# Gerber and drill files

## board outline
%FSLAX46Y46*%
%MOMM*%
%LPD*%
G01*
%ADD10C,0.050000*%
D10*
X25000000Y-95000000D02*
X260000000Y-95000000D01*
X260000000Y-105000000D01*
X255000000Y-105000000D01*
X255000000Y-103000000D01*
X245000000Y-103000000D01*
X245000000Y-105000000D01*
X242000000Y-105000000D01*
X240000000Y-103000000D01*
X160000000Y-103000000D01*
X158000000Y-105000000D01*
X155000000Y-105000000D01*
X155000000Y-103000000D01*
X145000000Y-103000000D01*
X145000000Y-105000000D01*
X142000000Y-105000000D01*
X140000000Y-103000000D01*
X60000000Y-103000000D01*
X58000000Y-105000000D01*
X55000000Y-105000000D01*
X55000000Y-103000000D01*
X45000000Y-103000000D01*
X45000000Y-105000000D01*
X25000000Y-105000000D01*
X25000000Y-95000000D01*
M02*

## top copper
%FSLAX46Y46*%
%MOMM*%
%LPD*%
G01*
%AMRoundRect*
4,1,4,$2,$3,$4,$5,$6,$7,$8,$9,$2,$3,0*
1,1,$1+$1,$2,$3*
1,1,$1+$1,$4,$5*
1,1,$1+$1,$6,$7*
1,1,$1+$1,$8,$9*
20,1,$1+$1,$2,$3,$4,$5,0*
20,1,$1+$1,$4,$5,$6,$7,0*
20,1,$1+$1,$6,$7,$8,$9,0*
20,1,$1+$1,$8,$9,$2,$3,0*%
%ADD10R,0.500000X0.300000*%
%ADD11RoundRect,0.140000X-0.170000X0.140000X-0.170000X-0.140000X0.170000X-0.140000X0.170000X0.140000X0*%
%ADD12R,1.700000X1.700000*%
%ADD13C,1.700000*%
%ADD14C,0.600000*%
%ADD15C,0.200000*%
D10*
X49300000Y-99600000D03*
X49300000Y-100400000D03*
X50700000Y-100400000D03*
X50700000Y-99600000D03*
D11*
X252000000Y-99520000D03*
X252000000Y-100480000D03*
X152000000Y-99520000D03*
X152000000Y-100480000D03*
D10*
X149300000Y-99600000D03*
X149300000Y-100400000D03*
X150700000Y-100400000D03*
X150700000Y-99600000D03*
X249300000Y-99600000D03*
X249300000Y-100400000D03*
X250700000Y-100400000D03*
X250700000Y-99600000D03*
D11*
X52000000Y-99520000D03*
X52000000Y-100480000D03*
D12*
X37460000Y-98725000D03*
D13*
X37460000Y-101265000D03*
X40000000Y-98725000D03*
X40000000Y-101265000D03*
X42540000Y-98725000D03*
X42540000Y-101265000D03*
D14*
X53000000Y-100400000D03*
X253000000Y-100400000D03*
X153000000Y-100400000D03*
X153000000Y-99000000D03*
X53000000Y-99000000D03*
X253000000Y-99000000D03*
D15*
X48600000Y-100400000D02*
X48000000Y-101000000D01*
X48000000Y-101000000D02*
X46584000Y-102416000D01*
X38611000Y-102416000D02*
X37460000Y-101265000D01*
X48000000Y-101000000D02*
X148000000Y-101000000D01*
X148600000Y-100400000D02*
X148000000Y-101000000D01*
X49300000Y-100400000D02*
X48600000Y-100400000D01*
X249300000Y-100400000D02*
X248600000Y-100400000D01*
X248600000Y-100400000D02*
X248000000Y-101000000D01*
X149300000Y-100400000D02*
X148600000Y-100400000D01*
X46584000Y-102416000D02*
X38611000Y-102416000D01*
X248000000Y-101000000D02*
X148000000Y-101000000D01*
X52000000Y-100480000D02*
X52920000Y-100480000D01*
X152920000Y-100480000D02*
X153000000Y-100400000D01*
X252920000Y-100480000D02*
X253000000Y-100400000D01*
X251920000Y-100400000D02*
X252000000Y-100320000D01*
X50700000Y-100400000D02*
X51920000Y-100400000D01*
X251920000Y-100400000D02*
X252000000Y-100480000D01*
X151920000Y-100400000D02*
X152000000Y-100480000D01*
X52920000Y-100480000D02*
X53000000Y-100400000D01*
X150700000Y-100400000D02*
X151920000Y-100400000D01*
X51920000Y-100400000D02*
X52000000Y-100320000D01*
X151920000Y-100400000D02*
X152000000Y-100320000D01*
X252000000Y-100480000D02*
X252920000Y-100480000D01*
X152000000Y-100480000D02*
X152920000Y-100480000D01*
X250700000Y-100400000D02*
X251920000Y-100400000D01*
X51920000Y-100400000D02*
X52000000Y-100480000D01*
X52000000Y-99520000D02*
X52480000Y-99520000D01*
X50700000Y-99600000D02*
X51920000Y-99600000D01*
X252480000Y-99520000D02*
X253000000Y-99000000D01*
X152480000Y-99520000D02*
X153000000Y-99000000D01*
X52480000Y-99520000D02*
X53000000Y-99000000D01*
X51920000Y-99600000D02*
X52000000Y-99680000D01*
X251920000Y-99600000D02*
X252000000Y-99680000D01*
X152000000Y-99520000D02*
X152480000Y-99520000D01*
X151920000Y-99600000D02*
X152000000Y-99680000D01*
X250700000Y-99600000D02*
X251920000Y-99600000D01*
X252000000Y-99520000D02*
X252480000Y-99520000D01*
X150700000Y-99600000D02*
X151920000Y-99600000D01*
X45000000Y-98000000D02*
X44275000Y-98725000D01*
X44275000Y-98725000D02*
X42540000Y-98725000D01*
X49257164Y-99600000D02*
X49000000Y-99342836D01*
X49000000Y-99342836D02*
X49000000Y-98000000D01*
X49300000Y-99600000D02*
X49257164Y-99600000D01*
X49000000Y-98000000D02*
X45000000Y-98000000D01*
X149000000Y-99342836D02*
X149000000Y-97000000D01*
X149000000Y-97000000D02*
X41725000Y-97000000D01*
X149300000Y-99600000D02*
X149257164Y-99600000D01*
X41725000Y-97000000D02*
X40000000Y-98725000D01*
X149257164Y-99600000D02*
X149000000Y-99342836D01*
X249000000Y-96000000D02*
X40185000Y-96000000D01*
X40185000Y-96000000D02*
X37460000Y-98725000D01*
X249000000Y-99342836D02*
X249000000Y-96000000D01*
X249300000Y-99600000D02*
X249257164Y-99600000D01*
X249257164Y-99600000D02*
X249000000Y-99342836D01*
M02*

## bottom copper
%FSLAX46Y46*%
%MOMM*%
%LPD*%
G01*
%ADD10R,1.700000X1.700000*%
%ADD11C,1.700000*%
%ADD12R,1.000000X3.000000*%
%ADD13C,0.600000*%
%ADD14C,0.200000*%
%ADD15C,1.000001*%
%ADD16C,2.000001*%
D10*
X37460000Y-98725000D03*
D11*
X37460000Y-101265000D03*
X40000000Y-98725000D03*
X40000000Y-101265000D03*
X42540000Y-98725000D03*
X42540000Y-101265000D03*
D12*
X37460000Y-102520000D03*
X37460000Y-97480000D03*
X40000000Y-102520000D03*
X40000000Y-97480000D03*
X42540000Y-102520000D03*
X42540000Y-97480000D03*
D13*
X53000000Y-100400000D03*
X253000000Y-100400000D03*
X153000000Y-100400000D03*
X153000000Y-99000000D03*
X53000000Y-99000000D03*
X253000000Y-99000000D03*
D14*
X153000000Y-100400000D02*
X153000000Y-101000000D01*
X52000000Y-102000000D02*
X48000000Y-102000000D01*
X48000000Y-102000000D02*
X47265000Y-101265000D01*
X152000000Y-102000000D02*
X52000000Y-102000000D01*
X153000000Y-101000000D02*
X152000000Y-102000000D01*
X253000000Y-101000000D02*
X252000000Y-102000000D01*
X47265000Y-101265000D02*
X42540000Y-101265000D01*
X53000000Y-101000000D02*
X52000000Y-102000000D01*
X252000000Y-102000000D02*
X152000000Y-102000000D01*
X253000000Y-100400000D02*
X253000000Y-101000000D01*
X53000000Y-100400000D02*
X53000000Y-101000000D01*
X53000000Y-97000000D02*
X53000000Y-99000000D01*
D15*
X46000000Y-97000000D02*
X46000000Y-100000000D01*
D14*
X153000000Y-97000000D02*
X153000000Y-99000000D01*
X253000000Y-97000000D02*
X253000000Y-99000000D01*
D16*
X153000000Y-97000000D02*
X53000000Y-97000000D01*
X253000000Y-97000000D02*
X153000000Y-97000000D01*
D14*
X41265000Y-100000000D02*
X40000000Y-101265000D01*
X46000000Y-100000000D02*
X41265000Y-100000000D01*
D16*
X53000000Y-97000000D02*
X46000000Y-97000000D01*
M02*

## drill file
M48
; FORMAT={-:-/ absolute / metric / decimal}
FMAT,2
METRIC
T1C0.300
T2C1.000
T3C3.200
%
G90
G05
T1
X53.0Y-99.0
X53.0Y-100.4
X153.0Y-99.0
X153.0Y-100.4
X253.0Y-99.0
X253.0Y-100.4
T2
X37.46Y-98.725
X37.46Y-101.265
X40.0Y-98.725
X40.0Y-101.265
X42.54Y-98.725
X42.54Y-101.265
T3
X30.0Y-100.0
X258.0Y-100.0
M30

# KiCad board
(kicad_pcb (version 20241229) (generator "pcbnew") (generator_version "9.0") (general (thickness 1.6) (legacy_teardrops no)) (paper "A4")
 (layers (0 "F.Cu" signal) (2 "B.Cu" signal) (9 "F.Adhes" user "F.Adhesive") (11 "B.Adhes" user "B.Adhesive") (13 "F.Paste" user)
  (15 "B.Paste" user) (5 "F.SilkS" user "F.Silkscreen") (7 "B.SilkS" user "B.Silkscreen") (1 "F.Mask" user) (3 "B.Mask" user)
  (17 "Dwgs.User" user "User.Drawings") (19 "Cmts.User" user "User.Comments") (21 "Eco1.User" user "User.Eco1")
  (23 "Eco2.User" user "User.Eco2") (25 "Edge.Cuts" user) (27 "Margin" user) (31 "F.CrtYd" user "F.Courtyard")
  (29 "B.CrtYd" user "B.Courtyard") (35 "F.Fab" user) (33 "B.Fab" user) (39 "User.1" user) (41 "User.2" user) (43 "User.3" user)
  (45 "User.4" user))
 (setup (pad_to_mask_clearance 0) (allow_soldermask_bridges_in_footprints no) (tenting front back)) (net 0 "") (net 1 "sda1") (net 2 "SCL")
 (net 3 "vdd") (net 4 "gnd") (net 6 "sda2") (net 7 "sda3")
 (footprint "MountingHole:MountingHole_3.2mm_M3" (layer "F.Cu") (at 258 100)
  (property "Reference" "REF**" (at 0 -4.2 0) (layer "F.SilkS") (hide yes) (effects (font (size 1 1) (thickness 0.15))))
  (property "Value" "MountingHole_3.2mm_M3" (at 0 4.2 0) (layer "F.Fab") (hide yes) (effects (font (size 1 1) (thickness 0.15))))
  (pad "" np_thru_hole circle (at 0 0) (size 3.2 3.2) (drill 3.2) (layers "*.Cu" "*.Mask")))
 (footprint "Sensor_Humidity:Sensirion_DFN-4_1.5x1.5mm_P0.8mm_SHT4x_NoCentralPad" (layer "F.Cu") (at 50 100)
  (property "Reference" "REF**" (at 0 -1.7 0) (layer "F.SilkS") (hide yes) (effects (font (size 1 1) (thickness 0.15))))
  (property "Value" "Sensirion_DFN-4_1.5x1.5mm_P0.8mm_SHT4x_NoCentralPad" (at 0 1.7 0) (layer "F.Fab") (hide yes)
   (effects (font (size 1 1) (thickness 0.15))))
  (pad "1" smd rect (at -0.7 -0.4) (size 0.5 0.3) (layers "F.Cu" "F.Mask" "F.Paste") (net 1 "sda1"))
  (pad "2" smd rect (at -0.7 0.4) (size 0.5 0.3) (layers "F.Cu" "F.Mask" "F.Paste") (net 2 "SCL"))
  (pad "3" smd rect (at 0.7 0.4) (size 0.5 0.3) (layers "F.Cu" "F.Mask" "F.Paste") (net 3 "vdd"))
  (pad "4" smd rect (at 0.7 -0.4) (size 0.5 0.3) (layers "F.Cu" "F.Mask" "F.Paste") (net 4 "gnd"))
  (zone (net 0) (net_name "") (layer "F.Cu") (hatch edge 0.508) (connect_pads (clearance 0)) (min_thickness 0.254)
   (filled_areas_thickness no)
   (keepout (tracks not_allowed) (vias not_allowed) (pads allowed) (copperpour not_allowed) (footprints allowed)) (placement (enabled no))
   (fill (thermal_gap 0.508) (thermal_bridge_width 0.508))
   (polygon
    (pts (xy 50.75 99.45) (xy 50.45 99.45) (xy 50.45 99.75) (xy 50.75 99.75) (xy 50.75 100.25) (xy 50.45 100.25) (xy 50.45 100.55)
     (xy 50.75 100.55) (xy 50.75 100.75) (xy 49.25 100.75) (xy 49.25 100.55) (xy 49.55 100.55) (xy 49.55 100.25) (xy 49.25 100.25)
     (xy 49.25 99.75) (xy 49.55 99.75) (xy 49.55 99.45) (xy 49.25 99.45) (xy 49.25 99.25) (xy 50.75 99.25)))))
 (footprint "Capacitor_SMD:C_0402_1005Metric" (layer "F.Cu") (at 252 100 -90)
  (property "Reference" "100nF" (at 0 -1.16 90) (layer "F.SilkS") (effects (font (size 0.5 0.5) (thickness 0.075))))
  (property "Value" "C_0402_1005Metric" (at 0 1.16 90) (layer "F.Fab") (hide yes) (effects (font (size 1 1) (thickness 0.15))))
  (pad "1" smd roundrect (at -0.48 0 270) (size 0.56 0.62) (layers "F.Cu" "F.Mask" "F.Paste") (roundrect_rratio 0.25) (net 4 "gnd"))
  (pad "2" smd roundrect (at 0.48 0 270) (size 0.56 0.62) (layers "F.Cu" "F.Mask" "F.Paste") (roundrect_rratio 0.25) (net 3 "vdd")))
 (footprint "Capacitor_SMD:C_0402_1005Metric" (layer "F.Cu") (at 152 100 -90)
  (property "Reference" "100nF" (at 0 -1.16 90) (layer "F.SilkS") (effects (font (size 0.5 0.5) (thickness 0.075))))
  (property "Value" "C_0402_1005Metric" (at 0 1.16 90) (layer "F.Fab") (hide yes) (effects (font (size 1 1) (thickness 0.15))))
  (pad "1" smd roundrect (at -0.48 0 270) (size 0.56 0.62) (layers "F.Cu" "F.Mask" "F.Paste") (roundrect_rratio 0.25) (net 4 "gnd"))
  (pad "2" smd roundrect (at 0.48 0 270) (size 0.56 0.62) (layers "F.Cu" "F.Mask" "F.Paste") (roundrect_rratio 0.25) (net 3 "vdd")))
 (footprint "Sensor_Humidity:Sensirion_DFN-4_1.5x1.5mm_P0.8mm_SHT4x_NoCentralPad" (layer "F.Cu") (at 150 100)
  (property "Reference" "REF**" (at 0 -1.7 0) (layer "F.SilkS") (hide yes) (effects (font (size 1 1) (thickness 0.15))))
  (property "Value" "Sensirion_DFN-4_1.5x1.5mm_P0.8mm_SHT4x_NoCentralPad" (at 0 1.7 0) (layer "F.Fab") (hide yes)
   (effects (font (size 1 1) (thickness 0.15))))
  (pad "1" smd rect (at -0.7 -0.4) (size 0.5 0.3) (layers "F.Cu" "F.Mask" "F.Paste") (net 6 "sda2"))
  (pad "2" smd rect (at -0.7 0.4) (size 0.5 0.3) (layers "F.Cu" "F.Mask" "F.Paste") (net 2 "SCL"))
  (pad "3" smd rect (at 0.7 0.4) (size 0.5 0.3) (layers "F.Cu" "F.Mask" "F.Paste"))
  (pad "4" smd rect (at 0.7 -0.4) (size 0.5 0.3) (layers "F.Cu" "F.Mask" "F.Paste"))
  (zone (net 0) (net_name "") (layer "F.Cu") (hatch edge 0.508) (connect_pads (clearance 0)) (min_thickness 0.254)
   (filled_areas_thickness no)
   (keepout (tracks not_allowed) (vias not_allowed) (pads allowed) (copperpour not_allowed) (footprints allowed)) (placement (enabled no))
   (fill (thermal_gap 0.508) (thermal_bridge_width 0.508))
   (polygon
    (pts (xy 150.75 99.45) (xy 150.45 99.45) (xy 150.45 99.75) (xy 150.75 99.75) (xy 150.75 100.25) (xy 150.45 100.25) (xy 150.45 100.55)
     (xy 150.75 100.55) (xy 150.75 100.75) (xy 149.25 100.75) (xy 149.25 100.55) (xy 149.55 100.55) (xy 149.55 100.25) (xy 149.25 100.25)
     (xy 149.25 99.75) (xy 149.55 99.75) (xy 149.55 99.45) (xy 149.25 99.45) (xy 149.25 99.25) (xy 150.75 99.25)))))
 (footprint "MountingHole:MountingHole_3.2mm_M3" (layer "F.Cu") (at 30 100)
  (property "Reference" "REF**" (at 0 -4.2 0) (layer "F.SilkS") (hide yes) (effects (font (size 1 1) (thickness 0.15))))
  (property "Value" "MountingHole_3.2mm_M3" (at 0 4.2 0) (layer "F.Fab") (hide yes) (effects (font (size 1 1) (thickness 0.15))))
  (pad "" np_thru_hole circle (at 0 0) (size 3.2 3.2) (drill 3.2) (layers "*.Cu" "*.Mask")))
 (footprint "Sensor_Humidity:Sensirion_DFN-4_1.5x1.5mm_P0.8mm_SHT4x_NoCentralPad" (layer "F.Cu") (at 250 100)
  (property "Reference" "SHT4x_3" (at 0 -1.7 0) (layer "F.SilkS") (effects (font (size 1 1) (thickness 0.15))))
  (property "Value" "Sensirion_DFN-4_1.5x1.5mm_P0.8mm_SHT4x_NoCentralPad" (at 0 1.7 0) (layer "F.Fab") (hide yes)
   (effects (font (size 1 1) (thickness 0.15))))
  (pad "1" smd rect (at -0.7 -0.4) (size 0.5 0.3) (layers "F.Cu" "F.Mask" "F.Paste") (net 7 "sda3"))
  (pad "2" smd rect (at -0.7 0.4) (size 0.5 0.3) (layers "F.Cu" "F.Mask" "F.Paste") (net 2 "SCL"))
  (pad "3" smd rect (at 0.7 0.4) (size 0.5 0.3) (layers "F.Cu" "F.Mask" "F.Paste") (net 3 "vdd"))
  (pad "4" smd rect (at 0.7 -0.4) (size 0.5 0.3) (layers "F.Cu" "F.Mask" "F.Paste"))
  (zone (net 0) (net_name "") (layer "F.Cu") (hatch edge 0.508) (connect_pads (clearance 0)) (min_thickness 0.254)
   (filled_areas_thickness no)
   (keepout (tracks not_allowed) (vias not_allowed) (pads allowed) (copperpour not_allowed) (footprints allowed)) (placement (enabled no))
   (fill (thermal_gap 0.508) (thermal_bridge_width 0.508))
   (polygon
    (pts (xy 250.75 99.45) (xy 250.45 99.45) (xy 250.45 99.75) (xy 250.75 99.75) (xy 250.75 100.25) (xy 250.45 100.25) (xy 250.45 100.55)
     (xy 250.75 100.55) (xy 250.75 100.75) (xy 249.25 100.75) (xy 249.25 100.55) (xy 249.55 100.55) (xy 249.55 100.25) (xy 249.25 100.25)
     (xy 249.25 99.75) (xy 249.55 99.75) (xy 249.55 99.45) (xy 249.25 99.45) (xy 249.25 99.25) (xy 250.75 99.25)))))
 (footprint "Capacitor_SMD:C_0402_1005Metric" (layer "F.Cu") (at 52 100 -90)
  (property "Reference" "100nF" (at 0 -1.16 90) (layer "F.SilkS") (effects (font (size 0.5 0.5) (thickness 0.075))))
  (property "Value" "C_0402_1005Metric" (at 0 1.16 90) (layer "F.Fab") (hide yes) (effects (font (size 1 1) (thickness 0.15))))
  (pad "1" smd roundrect (at -0.48 0 270) (size 0.56 0.62) (layers "F.Cu" "F.Mask" "F.Paste") (roundrect_rratio 0.25) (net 4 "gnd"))
  (pad "2" smd roundrect (at 0.48 0 270) (size 0.56 0.62) (layers "F.Cu" "F.Mask" "F.Paste") (roundrect_rratio 0.25) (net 3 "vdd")))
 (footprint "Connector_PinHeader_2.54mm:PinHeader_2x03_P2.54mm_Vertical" (layer "B.Cu") (at 37.46 98.725 -90)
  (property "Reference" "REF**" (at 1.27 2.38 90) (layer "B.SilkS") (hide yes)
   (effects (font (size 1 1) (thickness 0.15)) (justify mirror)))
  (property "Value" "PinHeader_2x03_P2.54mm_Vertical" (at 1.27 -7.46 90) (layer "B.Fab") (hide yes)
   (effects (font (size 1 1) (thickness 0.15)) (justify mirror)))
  (pad "1" thru_hole rect (at 0 0 270) (size 1.7 1.7) (drill 1) (layers "*.Cu" "B.Mask") (remove_unused_layers no) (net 7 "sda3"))
  (pad "2" thru_hole circle (at 2.54 0 270) (size 1.7 1.7) (drill 1) (layers "*.Cu" "B.Mask") (remove_unused_layers no) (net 2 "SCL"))
  (pad "3" thru_hole circle (at 0 -2.54 270) (size 1.7 1.7) (drill 1) (layers "*.Cu" "B.Mask") (remove_unused_layers no) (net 6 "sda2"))
  (pad "4" thru_hole circle (at 2.54 -2.54 270) (size 1.7 1.7) (drill 1) (layers "*.Cu" "B.Mask") (remove_unused_layers no) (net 4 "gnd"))
  (pad "5" thru_hole circle (at 0 -5.08 270) (size 1.7 1.7) (drill 1) (layers "*.Cu" "B.Mask") (remove_unused_layers no) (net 1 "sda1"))
  (pad "6" thru_hole circle (at 2.54 -5.08 270) (size 1.7 1.7) (drill 1) (layers "*.Cu" "B.Mask") (remove_unused_layers no) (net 3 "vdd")))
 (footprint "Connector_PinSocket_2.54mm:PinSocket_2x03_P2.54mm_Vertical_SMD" (layer "B.Cu") (at 40 100 -90)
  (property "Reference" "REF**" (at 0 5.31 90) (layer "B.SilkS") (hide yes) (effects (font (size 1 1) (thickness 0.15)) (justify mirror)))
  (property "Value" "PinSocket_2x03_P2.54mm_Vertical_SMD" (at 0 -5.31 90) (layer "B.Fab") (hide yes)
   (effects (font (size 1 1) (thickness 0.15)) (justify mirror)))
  (pad "1" smd rect (at 2.52 2.54 270) (size 3 1) (layers "B.Cu" "B.Mask" "B.Paste") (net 2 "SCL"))
  (pad "2" smd rect (at -2.52 2.54 270) (size 3 1) (layers "B.Cu" "B.Mask" "B.Paste") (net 7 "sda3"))
  (pad "3" smd rect (at 2.52 0 270) (size 3 1) (layers "B.Cu" "B.Mask" "B.Paste") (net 4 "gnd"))
  (pad "4" smd rect (at -2.52 0 270) (size 3 1) (layers "B.Cu" "B.Mask" "B.Paste") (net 6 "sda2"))
  (pad "5" smd rect (at 2.52 -2.54 270) (size 3 1) (layers "B.Cu" "B.Mask" "B.Paste") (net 3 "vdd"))
  (pad "6" smd rect (at -2.52 -2.54 270) (size 3 1) (layers "B.Cu" "B.Mask" "B.Paste") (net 1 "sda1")))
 (gr_poly
  (pts (xy 25 95) (xy 260 95) (xy 260 105) (xy 255 105) (xy 255 103) (xy 245 103) (xy 245 105) (xy 242 105) (xy 240 103) (xy 160 103)
   (xy 158 105) (xy 155 105) (xy 155 103) (xy 145 103) (xy 145 105) (xy 142 105) (xy 140 103) (xy 60 103) (xy 58 105) (xy 55 105)
   (xy 55 103) (xy 45 103) (xy 45 105) (xy 25 105))
  (stroke (width 0.05) (type solid)) (fill no) (layer "Edge.Cuts"))
 (segment (start 48.6 100.4) (end 48 101) (width 0.2) (layer "F.Cu") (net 2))
 (segment (start 48 101) (end 46.584 102.416) (width 0.2) (layer "F.Cu") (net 2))
 (segment (start 38.611 102.416) (end 37.46 101.265) (width 0.2) (layer "F.Cu") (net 2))
 (segment (start 48 101) (end 148 101) (width 0.2) (layer "F.Cu") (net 2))
 (segment (start 148.6 100.4) (end 148 101) (width 0.2) (layer "F.Cu") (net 2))
 (segment (start 49.3 100.4) (end 48.6 100.4) (width 0.2) (layer "F.Cu") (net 2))
 (segment (start 249.3 100.4) (end 248.6 100.4) (width 0.2) (layer "F.Cu") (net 2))
 (segment (start 248.6 100.4) (end 248 101) (width 0.2) (layer "F.Cu") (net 2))
 (segment (start 149.3 100.4) (end 148.6 100.4) (width 0.2) (layer "F.Cu") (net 2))
 (segment (start 46.584 102.416) (end 38.611 102.416) (width 0.2) (layer "F.Cu") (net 2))
 (segment (start 248 101) (end 148 101) (width 0.2) (layer "F.Cu") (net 2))
 (segment (start 52 100.48) (end 52.92 100.48) (width 0.2) (layer "F.Cu") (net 3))
 (segment (start 152.92 100.48) (end 153 100.4) (width 0.2) (layer "F.Cu") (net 3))
 (segment (start 252.92 100.48) (end 253 100.4) (width 0.2) (layer "F.Cu") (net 3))
 (segment (start 251.92 100.4) (end 252 100.32) (width 0.2) (layer "F.Cu") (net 3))
 (segment (start 50.7 100.4) (end 51.92 100.4) (width 0.2) (layer "F.Cu") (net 3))
 (segment (start 251.92 100.4) (end 252 100.48) (width 0.2) (layer "F.Cu") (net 3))
 (segment (start 151.92 100.4) (end 152 100.48) (width 0.2) (layer "F.Cu") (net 3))
 (segment (start 52.92 100.48) (end 53 100.4) (width 0.2) (layer "F.Cu") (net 3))
 (segment (start 150.7 100.4) (end 151.92 100.4) (width 0.2) (layer "F.Cu") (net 3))
 (segment (start 51.92 100.4) (end 52 100.32) (width 0.2) (layer "F.Cu") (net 3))
 (segment (start 151.92 100.4) (end 152 100.32) (width 0.2) (layer "F.Cu") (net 3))
 (segment (start 252 100.48) (end 252.92 100.48) (width 0.2) (layer "F.Cu") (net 3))
 (segment (start 152 100.48) (end 152.92 100.48) (width 0.2) (layer "F.Cu") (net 3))
 (segment (start 250.7 100.4) (end 251.92 100.4) (width 0.2) (layer "F.Cu") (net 3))
 (segment (start 51.92 100.4) (end 52 100.48) (width 0.2) (layer "F.Cu") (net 3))
 (via blind (at 53 100.4) (size 0.6) (drill 0.3) (layers "F.Cu" "B.Cu") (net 3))
 (via blind (at 253 100.4) (size 0.6) (drill 0.3) (layers "F.Cu" "B.Cu") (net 3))
 (via blind (at 153 100.4) (size 0.6) (drill 0.3) (layers "F.Cu" "B.Cu") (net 3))
 (segment (start 153 100.4) (end 153 101) (width 0.2) (layer "B.Cu") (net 3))
 (segment (start 52 102) (end 48 102) (width 0.2) (layer "B.Cu") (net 3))
 (segment (start 48 102) (end 47.265 101.265) (width 0.2) (layer "B.Cu") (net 3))
 (segment (start 152 102) (end 52 102) (width 0.2) (layer "B.Cu") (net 3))
 (segment (start 153 101) (end 152 102) (width 0.2) (layer "B.Cu") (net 3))
 (segment (start 253 101) (end 252 102) (width 0.2) (layer "B.Cu") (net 3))
 (segment (start 47.265 101.265) (end 42.54 101.265) (width 0.2) (layer "B.Cu") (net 3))
 (segment (start 53 101) (end 52 102) (width 0.2) (layer "B.Cu") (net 3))
 (segment (start 252 102) (end 152 102) (width 0.2) (layer "B.Cu") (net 3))
 (segment (start 253 100.4) (end 253 101) (width 0.2) (layer "B.Cu") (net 3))
 (segment (start 53 100.4) (end 53 101) (width 0.2) (layer "B.Cu") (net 3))
 (segment (start 52 99.52) (end 52.48 99.52) (width 0.2) (layer "F.Cu") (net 4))
 (segment (start 50.7 99.6) (end 51.92 99.6) (width 0.2) (layer "F.Cu") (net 4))
 (segment (start 252.48 99.52) (end 253 99) (width 0.2) (layer "F.Cu") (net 4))
 (segment (start 152.48 99.52) (end 153 99) (width 0.2) (layer "F.Cu") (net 4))
 (segment (start 52.48 99.52) (end 53 99) (width 0.2) (layer "F.Cu") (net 4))
 (segment (start 51.92 99.6) (end 52 99.68) (width 0.2) (layer "F.Cu") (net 4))
 (segment (start 251.92 99.6) (end 252 99.68) (width 0.2) (layer "F.Cu") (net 4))
 (segment (start 152 99.52) (end 152.48 99.52) (width 0.2) (layer "F.Cu") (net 4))
 (segment (start 151.92 99.6) (end 152 99.68) (width 0.2) (layer "F.Cu") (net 4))
 (segment (start 250.7 99.6) (end 251.92 99.6) (width 0.2) (layer "F.Cu") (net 4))
 (segment (start 252 99.52) (end 252.48 99.52) (width 0.2) (layer "F.Cu") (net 4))
 (segment (start 150.7 99.6) (end 151.92 99.6) (width 0.2) (layer "F.Cu") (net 4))
 (via blind (at 153 99) (size 0.6) (drill 0.3) (layers "F.Cu" "B.Cu") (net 4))
 (via blind (at 53 99) (size 0.6) (drill 0.3) (layers "F.Cu" "B.Cu") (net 4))
 (via blind (at 253 99) (size 0.6) (drill 0.3) (layers "F.Cu" "B.Cu") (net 4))
 (segment (start 53 97) (end 53 99) (width 0.2) (layer "B.Cu") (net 4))
 (segment (start 46 97) (end 46 100) (width 1.000001) (layer "B.Cu") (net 4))
 (segment (start 153 97) (end 153 99) (width 0.2) (layer "B.Cu") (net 4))
 (segment (start 253 97) (end 253 99) (width 0.2) (layer "B.Cu") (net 4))
 (segment (start 153 97) (end 53 97) (width 2.000001) (layer "B.Cu") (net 4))
 (segment (start 253 97) (end 153 97) (width 2.000001) (layer "B.Cu") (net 4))
 (segment (start 41.265 100) (end 40 101.265) (width 0.2) (layer "B.Cu") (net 4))
 (segment (start 46 100) (end 41.265 100) (width 0.2) (layer "B.Cu") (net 4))
 (segment (start 53 97) (end 46 97) (width 2.000001) (layer "B.Cu") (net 4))
 (segment (start 45 98) (end 44.275 98.725) (width 0.2) (layer "F.Cu") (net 1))
 (segment (start 44.275 98.725) (end 42.54 98.725) (width 0.2) (layer "F.Cu") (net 1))
 (segment (start 49.257164 99.6) (end 49 99.342836) (width 0.2) (layer "F.Cu") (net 1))
 (segment (start 49 99.342836) (end 49 98) (width 0.2) (layer "F.Cu") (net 1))
 (segment (start 49.3 99.6) (end 49.257164 99.6) (width 0.2) (layer "F.Cu") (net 1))
 (segment (start 49 98) (end 45 98) (width 0.2) (layer "F.Cu") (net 1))
 (segment (start 149 99.342836) (end 149 97) (width 0.2) (layer "F.Cu") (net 6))
 (segment (start 149 97) (end 41.725 97) (width 0.2) (layer "F.Cu") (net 6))
 (segment (start 149.3 99.6) (end 149.257164 99.6) (width 0.2) (layer "F.Cu") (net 6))
 (segment (start 41.725 97) (end 40 98.725) (width 0.2) (layer "F.Cu") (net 6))
 (segment (start 149.257164 99.6) (end 149 99.342836) (width 0.2) (layer "F.Cu") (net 6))
 (segment (start 249 96) (end 40.185 96) (width 0.2) (layer "F.Cu") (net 7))
 (segment (start 40.185 96) (end 37.46 98.725) (width 0.2) (layer "F.Cu") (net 7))
 (segment (start 249 99.342836) (end 249 96) (width 0.2) (layer "F.Cu") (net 7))
 (segment (start 249.3 99.6) (end 249.257164 99.6) (width 0.2) (layer "F.Cu") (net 7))
 (segment (start 249.257164 99.6) (end 249 99.342836) (width 0.2) (layer "F.Cu") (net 7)))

